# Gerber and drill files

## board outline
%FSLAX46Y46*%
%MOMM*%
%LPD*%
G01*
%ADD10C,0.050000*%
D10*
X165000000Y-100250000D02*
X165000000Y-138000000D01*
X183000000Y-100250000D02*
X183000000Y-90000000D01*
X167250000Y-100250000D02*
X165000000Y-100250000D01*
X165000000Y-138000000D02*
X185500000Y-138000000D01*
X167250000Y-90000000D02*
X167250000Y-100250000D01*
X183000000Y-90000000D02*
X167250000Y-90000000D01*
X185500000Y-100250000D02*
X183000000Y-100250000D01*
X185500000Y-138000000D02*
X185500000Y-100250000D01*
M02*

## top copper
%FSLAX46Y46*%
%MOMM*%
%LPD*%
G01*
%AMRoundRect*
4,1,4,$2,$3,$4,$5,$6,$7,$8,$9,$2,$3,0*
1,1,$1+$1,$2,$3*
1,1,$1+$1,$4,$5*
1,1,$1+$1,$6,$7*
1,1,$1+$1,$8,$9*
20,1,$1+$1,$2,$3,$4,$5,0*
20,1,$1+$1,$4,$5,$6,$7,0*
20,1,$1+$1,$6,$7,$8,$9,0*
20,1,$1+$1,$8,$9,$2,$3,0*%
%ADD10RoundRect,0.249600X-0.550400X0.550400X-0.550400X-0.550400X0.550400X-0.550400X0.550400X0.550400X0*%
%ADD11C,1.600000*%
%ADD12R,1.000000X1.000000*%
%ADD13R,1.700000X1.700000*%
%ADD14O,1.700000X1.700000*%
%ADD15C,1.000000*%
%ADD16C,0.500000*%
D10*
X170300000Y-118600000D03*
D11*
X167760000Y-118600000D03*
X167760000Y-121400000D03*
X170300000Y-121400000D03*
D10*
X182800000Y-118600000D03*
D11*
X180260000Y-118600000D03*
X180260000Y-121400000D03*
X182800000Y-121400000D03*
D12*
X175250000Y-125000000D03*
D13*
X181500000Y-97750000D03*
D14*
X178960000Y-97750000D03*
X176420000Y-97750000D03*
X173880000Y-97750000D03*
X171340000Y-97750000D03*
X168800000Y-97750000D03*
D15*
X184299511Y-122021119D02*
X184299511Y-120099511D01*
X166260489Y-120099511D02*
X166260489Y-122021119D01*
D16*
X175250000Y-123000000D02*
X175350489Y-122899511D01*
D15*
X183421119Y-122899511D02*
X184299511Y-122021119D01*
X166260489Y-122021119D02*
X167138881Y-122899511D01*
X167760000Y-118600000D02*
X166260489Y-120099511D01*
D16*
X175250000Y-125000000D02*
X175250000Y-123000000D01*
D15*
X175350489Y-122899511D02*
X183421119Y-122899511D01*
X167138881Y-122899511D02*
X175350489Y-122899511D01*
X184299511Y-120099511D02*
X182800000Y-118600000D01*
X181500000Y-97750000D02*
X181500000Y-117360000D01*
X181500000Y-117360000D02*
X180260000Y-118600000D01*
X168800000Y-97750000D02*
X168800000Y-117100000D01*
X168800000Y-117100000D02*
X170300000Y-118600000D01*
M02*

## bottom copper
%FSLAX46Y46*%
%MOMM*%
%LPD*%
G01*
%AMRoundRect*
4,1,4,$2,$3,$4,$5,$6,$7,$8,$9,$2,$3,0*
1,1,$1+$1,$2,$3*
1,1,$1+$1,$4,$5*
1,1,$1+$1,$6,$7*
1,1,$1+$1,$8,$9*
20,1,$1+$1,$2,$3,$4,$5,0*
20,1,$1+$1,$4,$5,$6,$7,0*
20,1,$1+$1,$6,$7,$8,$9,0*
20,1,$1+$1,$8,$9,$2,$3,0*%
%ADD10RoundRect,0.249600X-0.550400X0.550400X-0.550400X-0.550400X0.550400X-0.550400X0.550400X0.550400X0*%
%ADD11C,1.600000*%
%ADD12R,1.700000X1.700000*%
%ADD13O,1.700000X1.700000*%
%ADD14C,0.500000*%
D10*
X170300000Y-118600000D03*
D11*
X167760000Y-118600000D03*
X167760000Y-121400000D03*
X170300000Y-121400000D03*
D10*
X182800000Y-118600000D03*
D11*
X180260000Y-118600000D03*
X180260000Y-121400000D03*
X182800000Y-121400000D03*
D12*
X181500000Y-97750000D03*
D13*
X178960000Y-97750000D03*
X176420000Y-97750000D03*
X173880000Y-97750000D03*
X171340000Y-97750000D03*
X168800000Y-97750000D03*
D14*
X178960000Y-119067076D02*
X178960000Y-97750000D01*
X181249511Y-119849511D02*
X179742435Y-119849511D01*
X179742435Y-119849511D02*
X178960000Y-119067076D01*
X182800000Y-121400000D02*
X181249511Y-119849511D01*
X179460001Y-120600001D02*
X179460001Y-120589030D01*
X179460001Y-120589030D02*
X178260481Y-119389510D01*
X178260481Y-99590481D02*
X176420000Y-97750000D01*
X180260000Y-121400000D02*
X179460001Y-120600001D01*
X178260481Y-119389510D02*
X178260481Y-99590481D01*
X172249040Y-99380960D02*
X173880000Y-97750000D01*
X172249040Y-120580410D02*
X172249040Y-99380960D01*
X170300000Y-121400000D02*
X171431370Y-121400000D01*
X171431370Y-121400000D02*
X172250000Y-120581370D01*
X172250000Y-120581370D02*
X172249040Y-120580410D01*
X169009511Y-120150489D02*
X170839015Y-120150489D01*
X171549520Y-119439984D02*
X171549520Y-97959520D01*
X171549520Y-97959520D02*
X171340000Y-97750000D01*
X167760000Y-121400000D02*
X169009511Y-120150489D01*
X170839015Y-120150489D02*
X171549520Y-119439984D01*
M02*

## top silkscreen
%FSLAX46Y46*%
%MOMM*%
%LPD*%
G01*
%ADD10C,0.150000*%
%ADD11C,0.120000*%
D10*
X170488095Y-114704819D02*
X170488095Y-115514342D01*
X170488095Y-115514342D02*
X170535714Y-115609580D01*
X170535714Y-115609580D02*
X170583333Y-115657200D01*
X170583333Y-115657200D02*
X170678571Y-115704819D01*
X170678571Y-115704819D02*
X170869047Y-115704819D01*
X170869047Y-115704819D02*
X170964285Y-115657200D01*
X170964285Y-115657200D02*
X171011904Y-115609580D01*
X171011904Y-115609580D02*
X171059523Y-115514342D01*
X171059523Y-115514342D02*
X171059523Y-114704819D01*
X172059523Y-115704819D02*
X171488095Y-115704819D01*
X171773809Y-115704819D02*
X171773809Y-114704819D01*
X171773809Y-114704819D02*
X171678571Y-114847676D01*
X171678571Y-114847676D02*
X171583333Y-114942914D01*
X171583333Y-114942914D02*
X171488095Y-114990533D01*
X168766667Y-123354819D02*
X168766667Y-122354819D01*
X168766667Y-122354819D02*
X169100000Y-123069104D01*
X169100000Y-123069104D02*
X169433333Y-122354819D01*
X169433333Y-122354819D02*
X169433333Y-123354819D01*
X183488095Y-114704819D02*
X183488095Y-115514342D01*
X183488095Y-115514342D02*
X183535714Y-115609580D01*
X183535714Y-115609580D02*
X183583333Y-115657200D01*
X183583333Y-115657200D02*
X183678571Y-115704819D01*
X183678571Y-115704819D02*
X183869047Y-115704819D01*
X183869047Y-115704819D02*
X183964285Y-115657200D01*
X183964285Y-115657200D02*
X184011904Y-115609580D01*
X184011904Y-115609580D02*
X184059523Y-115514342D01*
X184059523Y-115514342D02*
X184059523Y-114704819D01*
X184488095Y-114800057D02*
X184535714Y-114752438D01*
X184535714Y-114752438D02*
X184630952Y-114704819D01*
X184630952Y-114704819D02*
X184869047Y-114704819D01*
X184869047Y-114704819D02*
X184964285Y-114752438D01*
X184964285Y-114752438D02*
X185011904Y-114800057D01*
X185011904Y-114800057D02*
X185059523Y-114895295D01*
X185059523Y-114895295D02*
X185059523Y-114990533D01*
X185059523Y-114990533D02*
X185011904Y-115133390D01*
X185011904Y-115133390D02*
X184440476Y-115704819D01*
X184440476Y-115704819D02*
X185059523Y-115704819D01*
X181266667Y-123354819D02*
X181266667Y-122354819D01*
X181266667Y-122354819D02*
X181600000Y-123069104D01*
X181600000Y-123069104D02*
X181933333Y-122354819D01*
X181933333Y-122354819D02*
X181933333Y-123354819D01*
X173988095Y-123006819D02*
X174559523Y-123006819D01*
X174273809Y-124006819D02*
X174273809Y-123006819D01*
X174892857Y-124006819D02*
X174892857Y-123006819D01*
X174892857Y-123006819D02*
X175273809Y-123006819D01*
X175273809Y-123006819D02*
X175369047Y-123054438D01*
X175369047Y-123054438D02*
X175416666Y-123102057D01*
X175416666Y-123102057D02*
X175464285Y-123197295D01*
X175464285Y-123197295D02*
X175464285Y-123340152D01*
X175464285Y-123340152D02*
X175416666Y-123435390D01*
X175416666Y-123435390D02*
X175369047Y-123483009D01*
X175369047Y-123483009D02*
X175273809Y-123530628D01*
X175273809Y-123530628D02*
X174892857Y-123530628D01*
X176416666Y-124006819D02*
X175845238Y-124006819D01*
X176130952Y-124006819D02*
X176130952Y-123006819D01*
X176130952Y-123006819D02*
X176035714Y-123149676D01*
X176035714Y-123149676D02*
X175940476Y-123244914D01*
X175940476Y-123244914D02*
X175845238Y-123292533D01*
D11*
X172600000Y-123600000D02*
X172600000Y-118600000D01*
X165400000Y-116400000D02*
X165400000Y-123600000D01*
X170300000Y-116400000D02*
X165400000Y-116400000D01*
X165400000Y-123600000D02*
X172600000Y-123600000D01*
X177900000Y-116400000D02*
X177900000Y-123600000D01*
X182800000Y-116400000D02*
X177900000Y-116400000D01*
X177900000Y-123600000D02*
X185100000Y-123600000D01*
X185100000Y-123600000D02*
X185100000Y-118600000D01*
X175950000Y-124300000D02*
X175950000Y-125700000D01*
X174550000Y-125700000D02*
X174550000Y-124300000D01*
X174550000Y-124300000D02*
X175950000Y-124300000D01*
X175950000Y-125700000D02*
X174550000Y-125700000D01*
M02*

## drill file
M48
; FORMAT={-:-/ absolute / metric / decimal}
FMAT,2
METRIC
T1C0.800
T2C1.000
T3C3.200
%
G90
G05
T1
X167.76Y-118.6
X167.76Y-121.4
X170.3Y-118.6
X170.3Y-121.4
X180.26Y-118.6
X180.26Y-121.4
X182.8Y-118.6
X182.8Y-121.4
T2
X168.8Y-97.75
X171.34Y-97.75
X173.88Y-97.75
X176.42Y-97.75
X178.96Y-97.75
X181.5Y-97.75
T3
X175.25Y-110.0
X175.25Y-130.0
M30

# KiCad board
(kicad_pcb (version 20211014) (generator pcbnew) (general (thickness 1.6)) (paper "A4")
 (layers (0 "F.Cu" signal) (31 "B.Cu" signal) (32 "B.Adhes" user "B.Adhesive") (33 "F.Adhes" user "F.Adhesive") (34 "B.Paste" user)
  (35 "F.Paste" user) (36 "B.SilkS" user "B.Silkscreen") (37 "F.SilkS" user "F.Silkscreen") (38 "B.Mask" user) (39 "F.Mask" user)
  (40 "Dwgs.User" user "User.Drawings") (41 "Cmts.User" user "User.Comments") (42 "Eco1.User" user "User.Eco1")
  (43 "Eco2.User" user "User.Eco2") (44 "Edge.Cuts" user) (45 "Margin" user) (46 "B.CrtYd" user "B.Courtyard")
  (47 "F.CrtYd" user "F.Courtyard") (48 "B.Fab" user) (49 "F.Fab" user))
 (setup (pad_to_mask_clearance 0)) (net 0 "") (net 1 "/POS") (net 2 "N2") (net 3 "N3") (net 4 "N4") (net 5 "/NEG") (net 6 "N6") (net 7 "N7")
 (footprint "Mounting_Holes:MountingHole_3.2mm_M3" (layer "F.Cu") (at 175.25 130)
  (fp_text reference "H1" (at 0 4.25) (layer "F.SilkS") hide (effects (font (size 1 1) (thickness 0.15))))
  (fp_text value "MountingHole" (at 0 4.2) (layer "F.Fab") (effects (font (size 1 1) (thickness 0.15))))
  (pad "" np_thru_hole circle locked (at 0 0) (size 3.2 3.2) (drill 3.2) (layers *.Cu *.Mask)))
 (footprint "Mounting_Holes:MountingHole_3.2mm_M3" (layer "F.Cu") (at 175.25 110)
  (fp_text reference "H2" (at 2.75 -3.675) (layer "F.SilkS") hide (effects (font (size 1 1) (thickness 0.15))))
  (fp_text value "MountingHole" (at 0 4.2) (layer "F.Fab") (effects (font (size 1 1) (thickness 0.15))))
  (pad "" np_thru_hole circle locked (at 0 0) (size 3.2 3.2) (drill 3.2) (layers *.Cu *.Mask)))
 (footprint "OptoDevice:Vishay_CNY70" (layer "F.Cu") (at 170.3 118.6 -90)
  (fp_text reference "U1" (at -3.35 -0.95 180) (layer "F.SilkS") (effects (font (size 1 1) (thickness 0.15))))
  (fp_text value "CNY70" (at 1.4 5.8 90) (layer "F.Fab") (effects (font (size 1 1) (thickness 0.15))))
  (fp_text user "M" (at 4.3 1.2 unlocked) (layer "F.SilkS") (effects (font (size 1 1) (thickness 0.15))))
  (fp_line (start 5 -2.3) (end 0 -2.3) (layer "F.SilkS") (width 0.12))
  (fp_line (start -2.2 4.9) (end 5 4.9) (layer "F.SilkS") (width 0.12))
  (fp_line (start -2.2 0) (end -2.2 4.9) (layer "F.SilkS") (width 0.12))
  (fp_line (start 5 4.9) (end 5 -2.3) (layer "F.SilkS") (width 0.12))
  (pad "1" thru_hole roundrect (at 0 0 270) (size 1.6 1.6) (drill 0.8) (layers *.Cu *.Mask) (roundrect_rratio 0.156) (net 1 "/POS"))
  (pad "2" thru_hole circle (at 0 2.54 270) (size 1.6 1.6) (drill 0.8) (layers *.Cu *.Mask) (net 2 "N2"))
  (pad "3" thru_hole circle (at 2.8 2.54 270) (size 1.6 1.6) (drill 0.8) (layers *.Cu *.Mask) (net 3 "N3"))
  (pad "4" thru_hole circle (at 2.8 0 270) (size 1.6 1.6) (drill 0.8) (layers *.Cu *.Mask) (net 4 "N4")))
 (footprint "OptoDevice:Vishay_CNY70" (layer "F.Cu") (at 182.8 118.6 -90)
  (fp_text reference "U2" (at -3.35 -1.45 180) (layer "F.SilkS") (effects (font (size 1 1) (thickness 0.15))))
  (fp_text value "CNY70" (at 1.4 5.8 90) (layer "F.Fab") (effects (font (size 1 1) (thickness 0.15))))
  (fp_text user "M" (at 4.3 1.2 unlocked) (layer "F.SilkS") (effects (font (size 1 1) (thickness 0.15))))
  (fp_line (start -2.2 4.9) (end 5 4.9) (layer "F.SilkS") (width 0.12))
  (fp_line (start -2.2 0) (end -2.2 4.9) (layer "F.SilkS") (width 0.12))
  (fp_line (start 5 4.9) (end 5 -2.3) (layer "F.SilkS") (width 0.12))
  (fp_line (start 5 -2.3) (end 0 -2.3) (layer "F.SilkS") (width 0.12))
  (pad "1" thru_hole roundrect (at 0 0 270) (size 1.6 1.6) (drill 0.8) (layers *.Cu *.Mask) (roundrect_rratio 0.156) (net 2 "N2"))
  (pad "2" thru_hole circle (at 0 2.54 270) (size 1.6 1.6) (drill 0.8) (layers *.Cu *.Mask) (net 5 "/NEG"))
  (pad "3" thru_hole circle (at 2.8 2.54 270) (size 1.6 1.6) (drill 0.8) (layers *.Cu *.Mask) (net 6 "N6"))
  (pad "4" thru_hole circle (at 2.8 0 270) (size 1.6 1.6) (drill 0.8) (layers *.Cu *.Mask) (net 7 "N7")))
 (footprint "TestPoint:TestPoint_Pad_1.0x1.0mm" (layer "F.Cu") (at 175.25 125)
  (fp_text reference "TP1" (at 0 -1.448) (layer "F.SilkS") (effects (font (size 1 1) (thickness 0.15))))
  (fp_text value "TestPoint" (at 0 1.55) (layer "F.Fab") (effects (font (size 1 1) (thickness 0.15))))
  (fp_line (start 0.7 -0.7) (end 0.7 0.7) (layer "F.SilkS") (width 0.12))
  (fp_line (start -0.7 0.7) (end -0.7 -0.7) (layer "F.SilkS") (width 0.12))
  (fp_line (start -0.7 -0.7) (end 0.7 -0.7) (layer "F.SilkS") (width 0.12))
  (fp_line (start 0.7 0.7) (end -0.7 0.7) (layer "F.SilkS") (width 0.12))
  (pad "1" smd rect locked (at 0 0) (size 1 1) (layers "F.Cu" "F.Mask") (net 2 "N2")))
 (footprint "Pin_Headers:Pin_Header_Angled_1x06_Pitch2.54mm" (layer "B.Cu") (at 181.5 97.75 90)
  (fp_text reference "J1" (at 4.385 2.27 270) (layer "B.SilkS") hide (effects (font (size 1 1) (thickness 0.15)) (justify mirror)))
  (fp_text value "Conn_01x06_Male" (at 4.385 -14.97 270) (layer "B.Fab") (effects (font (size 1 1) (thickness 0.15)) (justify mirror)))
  (pad "1" thru_hole rect (at 0 0 90) (size 1.7 1.7) (drill 1) (layers *.Cu *.Mask) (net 5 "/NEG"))
  (pad "2" thru_hole oval (at 0 -2.54 90) (size 1.7 1.7) (drill 1) (layers *.Cu *.Mask) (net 7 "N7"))
  (pad "3" thru_hole oval (at 0 -5.08 90) (size 1.7 1.7) (drill 1) (layers *.Cu *.Mask) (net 6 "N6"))
  (pad "4" thru_hole oval (at 0 -7.62 90) (size 1.7 1.7) (drill 1) (layers *.Cu *.Mask) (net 4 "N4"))
  (pad "5" thru_hole oval (at 0 -10.16 90) (size 1.7 1.7) (drill 1) (layers *.Cu *.Mask) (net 3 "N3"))
  (pad "6" thru_hole oval (at 0 -12.7 90) (size 1.7 1.7) (drill 1) (layers *.Cu *.Mask) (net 1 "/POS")))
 (gr_line (start 165 100.25) (end 165 138) (layer "Edge.Cuts") (width 0.05))
 (gr_line (start 183 100.25) (end 183 90) (layer "Edge.Cuts") (width 0.05))
 (gr_line (start 167.25 100.25) (end 165 100.25) (layer "Edge.Cuts") (width 0.05))
 (gr_line (start 165 138) (end 185.5 138) (layer "Edge.Cuts") (width 0.05))
 (gr_line (start 167.25 90) (end 167.25 100.25) (layer "Edge.Cuts") (width 0.05))
 (gr_line (start 183 90) (end 167.25 90) (layer "Edge.Cuts") (width 0.05))
 (gr_line (start 185.5 100.25) (end 183 100.25) (layer "Edge.Cuts") (width 0.05))
 (gr_line (start 185.5 138) (end 185.5 100.25) (layer "Edge.Cuts") (width 0.05))
 (segment (start 178.96 119.067076) (end 178.96 97.75) (width 0.5) (layer "B.Cu") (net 7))
 (segment (start 181.249511 119.849511) (end 179.742435 119.849511) (width 0.5) (layer "B.Cu") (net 7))
 (segment (start 179.742435 119.849511) (end 178.96 119.067076) (width 0.5) (layer "B.Cu") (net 7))
 (segment (start 182.8 121.4) (end 181.249511 119.849511) (width 0.5) (layer "B.Cu") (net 7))
 (segment (start 179.460001 120.600001) (end 179.460001 120.58903) (width 0.5) (layer "B.Cu") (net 6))
 (segment (start 179.460001 120.58903) (end 178.260481 119.38951) (width 0.5) (layer "B.Cu") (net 6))
 (segment (start 178.260481 99.590481) (end 176.42 97.75) (width 0.5) (layer "B.Cu") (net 6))
 (segment (start 180.26 121.4) (end 179.460001 120.600001) (width 0.5) (layer "B.Cu") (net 6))
 (segment (start 178.260481 119.38951) (end 178.260481 99.590481) (width 0.5) (layer "B.Cu") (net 6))
 (segment (start 172.24904 99.38096) (end 173.88 97.75) (width 0.5) (layer "B.Cu") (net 4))
 (segment (start 172.24904 120.58041) (end 172.24904 99.38096) (width 0.5) (layer "B.Cu") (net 4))
 (segment (start 170.3 121.4) (end 171.43137 121.4) (width 0.5) (layer "B.Cu") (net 4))
 (segment (start 171.43137 121.4) (end 172.25 120.58137) (width 0.5) (layer "B.Cu") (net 4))
 (segment (start 172.25 120.58137) (end 172.24904 120.58041) (width 0.5) (layer "B.Cu") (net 4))
 (segment (start 169.009511 120.150489) (end 170.839015 120.150489) (width 0.5) (layer "B.Cu") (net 3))
 (segment (start 171.54952 119.439984) (end 171.54952 97.95952) (width 0.5) (layer "B.Cu") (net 3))
 (segment (start 171.54952 97.95952) (end 171.34 97.75) (width 0.5) (layer "B.Cu") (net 3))
 (segment (start 167.76 121.4) (end 169.009511 120.150489) (width 0.5) (layer "B.Cu") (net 3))
 (segment (start 170.839015 120.150489) (end 171.54952 119.439984) (width 0.5) (layer "B.Cu") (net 3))
 (segment (start 184.299511 122.021119) (end 184.299511 120.099511) (width 1) (layer "F.Cu") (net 2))
 (segment (start 166.260489 120.099511) (end 166.260489 122.021119) (width 1) (layer "F.Cu") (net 2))
 (segment (start 175.25 123) (end 175.350489 122.899511) (width 0.5) (layer "F.Cu") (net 2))
 (segment (start 183.421119 122.899511) (end 184.299511 122.021119) (width 1) (layer "F.Cu") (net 2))
 (segment (start 166.260489 122.021119) (end 167.138881 122.899511) (width 1) (layer "F.Cu") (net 2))
 (segment (start 167.76 118.6) (end 166.260489 120.099511) (width 1) (layer "F.Cu") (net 2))
 (segment (start 175.25 125) (end 175.25 123) (width 0.5) (layer "F.Cu") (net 2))
 (segment (start 175.350489 122.899511) (end 183.421119 122.899511) (width 1) (layer "F.Cu") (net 2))
 (segment (start 167.138881 122.899511) (end 175.350489 122.899511) (width 1) (layer "F.Cu") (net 2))
 (segment (start 184.299511 120.099511) (end 182.8 118.6) (width 1) (layer "F.Cu") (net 2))
 (segment (start 181.5 97.75) (end 181.5 117.36) (width 1) (layer "F.Cu") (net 5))
 (segment (start 181.5 117.36) (end 180.26 118.6) (width 1) (layer "F.Cu") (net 5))
 (segment (start 168.8 97.75) (end 168.8 117.1) (width 1) (layer "F.Cu") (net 1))
 (segment (start 168.8 117.1) (end 170.3 118.6) (width 1) (layer "F.Cu") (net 1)))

